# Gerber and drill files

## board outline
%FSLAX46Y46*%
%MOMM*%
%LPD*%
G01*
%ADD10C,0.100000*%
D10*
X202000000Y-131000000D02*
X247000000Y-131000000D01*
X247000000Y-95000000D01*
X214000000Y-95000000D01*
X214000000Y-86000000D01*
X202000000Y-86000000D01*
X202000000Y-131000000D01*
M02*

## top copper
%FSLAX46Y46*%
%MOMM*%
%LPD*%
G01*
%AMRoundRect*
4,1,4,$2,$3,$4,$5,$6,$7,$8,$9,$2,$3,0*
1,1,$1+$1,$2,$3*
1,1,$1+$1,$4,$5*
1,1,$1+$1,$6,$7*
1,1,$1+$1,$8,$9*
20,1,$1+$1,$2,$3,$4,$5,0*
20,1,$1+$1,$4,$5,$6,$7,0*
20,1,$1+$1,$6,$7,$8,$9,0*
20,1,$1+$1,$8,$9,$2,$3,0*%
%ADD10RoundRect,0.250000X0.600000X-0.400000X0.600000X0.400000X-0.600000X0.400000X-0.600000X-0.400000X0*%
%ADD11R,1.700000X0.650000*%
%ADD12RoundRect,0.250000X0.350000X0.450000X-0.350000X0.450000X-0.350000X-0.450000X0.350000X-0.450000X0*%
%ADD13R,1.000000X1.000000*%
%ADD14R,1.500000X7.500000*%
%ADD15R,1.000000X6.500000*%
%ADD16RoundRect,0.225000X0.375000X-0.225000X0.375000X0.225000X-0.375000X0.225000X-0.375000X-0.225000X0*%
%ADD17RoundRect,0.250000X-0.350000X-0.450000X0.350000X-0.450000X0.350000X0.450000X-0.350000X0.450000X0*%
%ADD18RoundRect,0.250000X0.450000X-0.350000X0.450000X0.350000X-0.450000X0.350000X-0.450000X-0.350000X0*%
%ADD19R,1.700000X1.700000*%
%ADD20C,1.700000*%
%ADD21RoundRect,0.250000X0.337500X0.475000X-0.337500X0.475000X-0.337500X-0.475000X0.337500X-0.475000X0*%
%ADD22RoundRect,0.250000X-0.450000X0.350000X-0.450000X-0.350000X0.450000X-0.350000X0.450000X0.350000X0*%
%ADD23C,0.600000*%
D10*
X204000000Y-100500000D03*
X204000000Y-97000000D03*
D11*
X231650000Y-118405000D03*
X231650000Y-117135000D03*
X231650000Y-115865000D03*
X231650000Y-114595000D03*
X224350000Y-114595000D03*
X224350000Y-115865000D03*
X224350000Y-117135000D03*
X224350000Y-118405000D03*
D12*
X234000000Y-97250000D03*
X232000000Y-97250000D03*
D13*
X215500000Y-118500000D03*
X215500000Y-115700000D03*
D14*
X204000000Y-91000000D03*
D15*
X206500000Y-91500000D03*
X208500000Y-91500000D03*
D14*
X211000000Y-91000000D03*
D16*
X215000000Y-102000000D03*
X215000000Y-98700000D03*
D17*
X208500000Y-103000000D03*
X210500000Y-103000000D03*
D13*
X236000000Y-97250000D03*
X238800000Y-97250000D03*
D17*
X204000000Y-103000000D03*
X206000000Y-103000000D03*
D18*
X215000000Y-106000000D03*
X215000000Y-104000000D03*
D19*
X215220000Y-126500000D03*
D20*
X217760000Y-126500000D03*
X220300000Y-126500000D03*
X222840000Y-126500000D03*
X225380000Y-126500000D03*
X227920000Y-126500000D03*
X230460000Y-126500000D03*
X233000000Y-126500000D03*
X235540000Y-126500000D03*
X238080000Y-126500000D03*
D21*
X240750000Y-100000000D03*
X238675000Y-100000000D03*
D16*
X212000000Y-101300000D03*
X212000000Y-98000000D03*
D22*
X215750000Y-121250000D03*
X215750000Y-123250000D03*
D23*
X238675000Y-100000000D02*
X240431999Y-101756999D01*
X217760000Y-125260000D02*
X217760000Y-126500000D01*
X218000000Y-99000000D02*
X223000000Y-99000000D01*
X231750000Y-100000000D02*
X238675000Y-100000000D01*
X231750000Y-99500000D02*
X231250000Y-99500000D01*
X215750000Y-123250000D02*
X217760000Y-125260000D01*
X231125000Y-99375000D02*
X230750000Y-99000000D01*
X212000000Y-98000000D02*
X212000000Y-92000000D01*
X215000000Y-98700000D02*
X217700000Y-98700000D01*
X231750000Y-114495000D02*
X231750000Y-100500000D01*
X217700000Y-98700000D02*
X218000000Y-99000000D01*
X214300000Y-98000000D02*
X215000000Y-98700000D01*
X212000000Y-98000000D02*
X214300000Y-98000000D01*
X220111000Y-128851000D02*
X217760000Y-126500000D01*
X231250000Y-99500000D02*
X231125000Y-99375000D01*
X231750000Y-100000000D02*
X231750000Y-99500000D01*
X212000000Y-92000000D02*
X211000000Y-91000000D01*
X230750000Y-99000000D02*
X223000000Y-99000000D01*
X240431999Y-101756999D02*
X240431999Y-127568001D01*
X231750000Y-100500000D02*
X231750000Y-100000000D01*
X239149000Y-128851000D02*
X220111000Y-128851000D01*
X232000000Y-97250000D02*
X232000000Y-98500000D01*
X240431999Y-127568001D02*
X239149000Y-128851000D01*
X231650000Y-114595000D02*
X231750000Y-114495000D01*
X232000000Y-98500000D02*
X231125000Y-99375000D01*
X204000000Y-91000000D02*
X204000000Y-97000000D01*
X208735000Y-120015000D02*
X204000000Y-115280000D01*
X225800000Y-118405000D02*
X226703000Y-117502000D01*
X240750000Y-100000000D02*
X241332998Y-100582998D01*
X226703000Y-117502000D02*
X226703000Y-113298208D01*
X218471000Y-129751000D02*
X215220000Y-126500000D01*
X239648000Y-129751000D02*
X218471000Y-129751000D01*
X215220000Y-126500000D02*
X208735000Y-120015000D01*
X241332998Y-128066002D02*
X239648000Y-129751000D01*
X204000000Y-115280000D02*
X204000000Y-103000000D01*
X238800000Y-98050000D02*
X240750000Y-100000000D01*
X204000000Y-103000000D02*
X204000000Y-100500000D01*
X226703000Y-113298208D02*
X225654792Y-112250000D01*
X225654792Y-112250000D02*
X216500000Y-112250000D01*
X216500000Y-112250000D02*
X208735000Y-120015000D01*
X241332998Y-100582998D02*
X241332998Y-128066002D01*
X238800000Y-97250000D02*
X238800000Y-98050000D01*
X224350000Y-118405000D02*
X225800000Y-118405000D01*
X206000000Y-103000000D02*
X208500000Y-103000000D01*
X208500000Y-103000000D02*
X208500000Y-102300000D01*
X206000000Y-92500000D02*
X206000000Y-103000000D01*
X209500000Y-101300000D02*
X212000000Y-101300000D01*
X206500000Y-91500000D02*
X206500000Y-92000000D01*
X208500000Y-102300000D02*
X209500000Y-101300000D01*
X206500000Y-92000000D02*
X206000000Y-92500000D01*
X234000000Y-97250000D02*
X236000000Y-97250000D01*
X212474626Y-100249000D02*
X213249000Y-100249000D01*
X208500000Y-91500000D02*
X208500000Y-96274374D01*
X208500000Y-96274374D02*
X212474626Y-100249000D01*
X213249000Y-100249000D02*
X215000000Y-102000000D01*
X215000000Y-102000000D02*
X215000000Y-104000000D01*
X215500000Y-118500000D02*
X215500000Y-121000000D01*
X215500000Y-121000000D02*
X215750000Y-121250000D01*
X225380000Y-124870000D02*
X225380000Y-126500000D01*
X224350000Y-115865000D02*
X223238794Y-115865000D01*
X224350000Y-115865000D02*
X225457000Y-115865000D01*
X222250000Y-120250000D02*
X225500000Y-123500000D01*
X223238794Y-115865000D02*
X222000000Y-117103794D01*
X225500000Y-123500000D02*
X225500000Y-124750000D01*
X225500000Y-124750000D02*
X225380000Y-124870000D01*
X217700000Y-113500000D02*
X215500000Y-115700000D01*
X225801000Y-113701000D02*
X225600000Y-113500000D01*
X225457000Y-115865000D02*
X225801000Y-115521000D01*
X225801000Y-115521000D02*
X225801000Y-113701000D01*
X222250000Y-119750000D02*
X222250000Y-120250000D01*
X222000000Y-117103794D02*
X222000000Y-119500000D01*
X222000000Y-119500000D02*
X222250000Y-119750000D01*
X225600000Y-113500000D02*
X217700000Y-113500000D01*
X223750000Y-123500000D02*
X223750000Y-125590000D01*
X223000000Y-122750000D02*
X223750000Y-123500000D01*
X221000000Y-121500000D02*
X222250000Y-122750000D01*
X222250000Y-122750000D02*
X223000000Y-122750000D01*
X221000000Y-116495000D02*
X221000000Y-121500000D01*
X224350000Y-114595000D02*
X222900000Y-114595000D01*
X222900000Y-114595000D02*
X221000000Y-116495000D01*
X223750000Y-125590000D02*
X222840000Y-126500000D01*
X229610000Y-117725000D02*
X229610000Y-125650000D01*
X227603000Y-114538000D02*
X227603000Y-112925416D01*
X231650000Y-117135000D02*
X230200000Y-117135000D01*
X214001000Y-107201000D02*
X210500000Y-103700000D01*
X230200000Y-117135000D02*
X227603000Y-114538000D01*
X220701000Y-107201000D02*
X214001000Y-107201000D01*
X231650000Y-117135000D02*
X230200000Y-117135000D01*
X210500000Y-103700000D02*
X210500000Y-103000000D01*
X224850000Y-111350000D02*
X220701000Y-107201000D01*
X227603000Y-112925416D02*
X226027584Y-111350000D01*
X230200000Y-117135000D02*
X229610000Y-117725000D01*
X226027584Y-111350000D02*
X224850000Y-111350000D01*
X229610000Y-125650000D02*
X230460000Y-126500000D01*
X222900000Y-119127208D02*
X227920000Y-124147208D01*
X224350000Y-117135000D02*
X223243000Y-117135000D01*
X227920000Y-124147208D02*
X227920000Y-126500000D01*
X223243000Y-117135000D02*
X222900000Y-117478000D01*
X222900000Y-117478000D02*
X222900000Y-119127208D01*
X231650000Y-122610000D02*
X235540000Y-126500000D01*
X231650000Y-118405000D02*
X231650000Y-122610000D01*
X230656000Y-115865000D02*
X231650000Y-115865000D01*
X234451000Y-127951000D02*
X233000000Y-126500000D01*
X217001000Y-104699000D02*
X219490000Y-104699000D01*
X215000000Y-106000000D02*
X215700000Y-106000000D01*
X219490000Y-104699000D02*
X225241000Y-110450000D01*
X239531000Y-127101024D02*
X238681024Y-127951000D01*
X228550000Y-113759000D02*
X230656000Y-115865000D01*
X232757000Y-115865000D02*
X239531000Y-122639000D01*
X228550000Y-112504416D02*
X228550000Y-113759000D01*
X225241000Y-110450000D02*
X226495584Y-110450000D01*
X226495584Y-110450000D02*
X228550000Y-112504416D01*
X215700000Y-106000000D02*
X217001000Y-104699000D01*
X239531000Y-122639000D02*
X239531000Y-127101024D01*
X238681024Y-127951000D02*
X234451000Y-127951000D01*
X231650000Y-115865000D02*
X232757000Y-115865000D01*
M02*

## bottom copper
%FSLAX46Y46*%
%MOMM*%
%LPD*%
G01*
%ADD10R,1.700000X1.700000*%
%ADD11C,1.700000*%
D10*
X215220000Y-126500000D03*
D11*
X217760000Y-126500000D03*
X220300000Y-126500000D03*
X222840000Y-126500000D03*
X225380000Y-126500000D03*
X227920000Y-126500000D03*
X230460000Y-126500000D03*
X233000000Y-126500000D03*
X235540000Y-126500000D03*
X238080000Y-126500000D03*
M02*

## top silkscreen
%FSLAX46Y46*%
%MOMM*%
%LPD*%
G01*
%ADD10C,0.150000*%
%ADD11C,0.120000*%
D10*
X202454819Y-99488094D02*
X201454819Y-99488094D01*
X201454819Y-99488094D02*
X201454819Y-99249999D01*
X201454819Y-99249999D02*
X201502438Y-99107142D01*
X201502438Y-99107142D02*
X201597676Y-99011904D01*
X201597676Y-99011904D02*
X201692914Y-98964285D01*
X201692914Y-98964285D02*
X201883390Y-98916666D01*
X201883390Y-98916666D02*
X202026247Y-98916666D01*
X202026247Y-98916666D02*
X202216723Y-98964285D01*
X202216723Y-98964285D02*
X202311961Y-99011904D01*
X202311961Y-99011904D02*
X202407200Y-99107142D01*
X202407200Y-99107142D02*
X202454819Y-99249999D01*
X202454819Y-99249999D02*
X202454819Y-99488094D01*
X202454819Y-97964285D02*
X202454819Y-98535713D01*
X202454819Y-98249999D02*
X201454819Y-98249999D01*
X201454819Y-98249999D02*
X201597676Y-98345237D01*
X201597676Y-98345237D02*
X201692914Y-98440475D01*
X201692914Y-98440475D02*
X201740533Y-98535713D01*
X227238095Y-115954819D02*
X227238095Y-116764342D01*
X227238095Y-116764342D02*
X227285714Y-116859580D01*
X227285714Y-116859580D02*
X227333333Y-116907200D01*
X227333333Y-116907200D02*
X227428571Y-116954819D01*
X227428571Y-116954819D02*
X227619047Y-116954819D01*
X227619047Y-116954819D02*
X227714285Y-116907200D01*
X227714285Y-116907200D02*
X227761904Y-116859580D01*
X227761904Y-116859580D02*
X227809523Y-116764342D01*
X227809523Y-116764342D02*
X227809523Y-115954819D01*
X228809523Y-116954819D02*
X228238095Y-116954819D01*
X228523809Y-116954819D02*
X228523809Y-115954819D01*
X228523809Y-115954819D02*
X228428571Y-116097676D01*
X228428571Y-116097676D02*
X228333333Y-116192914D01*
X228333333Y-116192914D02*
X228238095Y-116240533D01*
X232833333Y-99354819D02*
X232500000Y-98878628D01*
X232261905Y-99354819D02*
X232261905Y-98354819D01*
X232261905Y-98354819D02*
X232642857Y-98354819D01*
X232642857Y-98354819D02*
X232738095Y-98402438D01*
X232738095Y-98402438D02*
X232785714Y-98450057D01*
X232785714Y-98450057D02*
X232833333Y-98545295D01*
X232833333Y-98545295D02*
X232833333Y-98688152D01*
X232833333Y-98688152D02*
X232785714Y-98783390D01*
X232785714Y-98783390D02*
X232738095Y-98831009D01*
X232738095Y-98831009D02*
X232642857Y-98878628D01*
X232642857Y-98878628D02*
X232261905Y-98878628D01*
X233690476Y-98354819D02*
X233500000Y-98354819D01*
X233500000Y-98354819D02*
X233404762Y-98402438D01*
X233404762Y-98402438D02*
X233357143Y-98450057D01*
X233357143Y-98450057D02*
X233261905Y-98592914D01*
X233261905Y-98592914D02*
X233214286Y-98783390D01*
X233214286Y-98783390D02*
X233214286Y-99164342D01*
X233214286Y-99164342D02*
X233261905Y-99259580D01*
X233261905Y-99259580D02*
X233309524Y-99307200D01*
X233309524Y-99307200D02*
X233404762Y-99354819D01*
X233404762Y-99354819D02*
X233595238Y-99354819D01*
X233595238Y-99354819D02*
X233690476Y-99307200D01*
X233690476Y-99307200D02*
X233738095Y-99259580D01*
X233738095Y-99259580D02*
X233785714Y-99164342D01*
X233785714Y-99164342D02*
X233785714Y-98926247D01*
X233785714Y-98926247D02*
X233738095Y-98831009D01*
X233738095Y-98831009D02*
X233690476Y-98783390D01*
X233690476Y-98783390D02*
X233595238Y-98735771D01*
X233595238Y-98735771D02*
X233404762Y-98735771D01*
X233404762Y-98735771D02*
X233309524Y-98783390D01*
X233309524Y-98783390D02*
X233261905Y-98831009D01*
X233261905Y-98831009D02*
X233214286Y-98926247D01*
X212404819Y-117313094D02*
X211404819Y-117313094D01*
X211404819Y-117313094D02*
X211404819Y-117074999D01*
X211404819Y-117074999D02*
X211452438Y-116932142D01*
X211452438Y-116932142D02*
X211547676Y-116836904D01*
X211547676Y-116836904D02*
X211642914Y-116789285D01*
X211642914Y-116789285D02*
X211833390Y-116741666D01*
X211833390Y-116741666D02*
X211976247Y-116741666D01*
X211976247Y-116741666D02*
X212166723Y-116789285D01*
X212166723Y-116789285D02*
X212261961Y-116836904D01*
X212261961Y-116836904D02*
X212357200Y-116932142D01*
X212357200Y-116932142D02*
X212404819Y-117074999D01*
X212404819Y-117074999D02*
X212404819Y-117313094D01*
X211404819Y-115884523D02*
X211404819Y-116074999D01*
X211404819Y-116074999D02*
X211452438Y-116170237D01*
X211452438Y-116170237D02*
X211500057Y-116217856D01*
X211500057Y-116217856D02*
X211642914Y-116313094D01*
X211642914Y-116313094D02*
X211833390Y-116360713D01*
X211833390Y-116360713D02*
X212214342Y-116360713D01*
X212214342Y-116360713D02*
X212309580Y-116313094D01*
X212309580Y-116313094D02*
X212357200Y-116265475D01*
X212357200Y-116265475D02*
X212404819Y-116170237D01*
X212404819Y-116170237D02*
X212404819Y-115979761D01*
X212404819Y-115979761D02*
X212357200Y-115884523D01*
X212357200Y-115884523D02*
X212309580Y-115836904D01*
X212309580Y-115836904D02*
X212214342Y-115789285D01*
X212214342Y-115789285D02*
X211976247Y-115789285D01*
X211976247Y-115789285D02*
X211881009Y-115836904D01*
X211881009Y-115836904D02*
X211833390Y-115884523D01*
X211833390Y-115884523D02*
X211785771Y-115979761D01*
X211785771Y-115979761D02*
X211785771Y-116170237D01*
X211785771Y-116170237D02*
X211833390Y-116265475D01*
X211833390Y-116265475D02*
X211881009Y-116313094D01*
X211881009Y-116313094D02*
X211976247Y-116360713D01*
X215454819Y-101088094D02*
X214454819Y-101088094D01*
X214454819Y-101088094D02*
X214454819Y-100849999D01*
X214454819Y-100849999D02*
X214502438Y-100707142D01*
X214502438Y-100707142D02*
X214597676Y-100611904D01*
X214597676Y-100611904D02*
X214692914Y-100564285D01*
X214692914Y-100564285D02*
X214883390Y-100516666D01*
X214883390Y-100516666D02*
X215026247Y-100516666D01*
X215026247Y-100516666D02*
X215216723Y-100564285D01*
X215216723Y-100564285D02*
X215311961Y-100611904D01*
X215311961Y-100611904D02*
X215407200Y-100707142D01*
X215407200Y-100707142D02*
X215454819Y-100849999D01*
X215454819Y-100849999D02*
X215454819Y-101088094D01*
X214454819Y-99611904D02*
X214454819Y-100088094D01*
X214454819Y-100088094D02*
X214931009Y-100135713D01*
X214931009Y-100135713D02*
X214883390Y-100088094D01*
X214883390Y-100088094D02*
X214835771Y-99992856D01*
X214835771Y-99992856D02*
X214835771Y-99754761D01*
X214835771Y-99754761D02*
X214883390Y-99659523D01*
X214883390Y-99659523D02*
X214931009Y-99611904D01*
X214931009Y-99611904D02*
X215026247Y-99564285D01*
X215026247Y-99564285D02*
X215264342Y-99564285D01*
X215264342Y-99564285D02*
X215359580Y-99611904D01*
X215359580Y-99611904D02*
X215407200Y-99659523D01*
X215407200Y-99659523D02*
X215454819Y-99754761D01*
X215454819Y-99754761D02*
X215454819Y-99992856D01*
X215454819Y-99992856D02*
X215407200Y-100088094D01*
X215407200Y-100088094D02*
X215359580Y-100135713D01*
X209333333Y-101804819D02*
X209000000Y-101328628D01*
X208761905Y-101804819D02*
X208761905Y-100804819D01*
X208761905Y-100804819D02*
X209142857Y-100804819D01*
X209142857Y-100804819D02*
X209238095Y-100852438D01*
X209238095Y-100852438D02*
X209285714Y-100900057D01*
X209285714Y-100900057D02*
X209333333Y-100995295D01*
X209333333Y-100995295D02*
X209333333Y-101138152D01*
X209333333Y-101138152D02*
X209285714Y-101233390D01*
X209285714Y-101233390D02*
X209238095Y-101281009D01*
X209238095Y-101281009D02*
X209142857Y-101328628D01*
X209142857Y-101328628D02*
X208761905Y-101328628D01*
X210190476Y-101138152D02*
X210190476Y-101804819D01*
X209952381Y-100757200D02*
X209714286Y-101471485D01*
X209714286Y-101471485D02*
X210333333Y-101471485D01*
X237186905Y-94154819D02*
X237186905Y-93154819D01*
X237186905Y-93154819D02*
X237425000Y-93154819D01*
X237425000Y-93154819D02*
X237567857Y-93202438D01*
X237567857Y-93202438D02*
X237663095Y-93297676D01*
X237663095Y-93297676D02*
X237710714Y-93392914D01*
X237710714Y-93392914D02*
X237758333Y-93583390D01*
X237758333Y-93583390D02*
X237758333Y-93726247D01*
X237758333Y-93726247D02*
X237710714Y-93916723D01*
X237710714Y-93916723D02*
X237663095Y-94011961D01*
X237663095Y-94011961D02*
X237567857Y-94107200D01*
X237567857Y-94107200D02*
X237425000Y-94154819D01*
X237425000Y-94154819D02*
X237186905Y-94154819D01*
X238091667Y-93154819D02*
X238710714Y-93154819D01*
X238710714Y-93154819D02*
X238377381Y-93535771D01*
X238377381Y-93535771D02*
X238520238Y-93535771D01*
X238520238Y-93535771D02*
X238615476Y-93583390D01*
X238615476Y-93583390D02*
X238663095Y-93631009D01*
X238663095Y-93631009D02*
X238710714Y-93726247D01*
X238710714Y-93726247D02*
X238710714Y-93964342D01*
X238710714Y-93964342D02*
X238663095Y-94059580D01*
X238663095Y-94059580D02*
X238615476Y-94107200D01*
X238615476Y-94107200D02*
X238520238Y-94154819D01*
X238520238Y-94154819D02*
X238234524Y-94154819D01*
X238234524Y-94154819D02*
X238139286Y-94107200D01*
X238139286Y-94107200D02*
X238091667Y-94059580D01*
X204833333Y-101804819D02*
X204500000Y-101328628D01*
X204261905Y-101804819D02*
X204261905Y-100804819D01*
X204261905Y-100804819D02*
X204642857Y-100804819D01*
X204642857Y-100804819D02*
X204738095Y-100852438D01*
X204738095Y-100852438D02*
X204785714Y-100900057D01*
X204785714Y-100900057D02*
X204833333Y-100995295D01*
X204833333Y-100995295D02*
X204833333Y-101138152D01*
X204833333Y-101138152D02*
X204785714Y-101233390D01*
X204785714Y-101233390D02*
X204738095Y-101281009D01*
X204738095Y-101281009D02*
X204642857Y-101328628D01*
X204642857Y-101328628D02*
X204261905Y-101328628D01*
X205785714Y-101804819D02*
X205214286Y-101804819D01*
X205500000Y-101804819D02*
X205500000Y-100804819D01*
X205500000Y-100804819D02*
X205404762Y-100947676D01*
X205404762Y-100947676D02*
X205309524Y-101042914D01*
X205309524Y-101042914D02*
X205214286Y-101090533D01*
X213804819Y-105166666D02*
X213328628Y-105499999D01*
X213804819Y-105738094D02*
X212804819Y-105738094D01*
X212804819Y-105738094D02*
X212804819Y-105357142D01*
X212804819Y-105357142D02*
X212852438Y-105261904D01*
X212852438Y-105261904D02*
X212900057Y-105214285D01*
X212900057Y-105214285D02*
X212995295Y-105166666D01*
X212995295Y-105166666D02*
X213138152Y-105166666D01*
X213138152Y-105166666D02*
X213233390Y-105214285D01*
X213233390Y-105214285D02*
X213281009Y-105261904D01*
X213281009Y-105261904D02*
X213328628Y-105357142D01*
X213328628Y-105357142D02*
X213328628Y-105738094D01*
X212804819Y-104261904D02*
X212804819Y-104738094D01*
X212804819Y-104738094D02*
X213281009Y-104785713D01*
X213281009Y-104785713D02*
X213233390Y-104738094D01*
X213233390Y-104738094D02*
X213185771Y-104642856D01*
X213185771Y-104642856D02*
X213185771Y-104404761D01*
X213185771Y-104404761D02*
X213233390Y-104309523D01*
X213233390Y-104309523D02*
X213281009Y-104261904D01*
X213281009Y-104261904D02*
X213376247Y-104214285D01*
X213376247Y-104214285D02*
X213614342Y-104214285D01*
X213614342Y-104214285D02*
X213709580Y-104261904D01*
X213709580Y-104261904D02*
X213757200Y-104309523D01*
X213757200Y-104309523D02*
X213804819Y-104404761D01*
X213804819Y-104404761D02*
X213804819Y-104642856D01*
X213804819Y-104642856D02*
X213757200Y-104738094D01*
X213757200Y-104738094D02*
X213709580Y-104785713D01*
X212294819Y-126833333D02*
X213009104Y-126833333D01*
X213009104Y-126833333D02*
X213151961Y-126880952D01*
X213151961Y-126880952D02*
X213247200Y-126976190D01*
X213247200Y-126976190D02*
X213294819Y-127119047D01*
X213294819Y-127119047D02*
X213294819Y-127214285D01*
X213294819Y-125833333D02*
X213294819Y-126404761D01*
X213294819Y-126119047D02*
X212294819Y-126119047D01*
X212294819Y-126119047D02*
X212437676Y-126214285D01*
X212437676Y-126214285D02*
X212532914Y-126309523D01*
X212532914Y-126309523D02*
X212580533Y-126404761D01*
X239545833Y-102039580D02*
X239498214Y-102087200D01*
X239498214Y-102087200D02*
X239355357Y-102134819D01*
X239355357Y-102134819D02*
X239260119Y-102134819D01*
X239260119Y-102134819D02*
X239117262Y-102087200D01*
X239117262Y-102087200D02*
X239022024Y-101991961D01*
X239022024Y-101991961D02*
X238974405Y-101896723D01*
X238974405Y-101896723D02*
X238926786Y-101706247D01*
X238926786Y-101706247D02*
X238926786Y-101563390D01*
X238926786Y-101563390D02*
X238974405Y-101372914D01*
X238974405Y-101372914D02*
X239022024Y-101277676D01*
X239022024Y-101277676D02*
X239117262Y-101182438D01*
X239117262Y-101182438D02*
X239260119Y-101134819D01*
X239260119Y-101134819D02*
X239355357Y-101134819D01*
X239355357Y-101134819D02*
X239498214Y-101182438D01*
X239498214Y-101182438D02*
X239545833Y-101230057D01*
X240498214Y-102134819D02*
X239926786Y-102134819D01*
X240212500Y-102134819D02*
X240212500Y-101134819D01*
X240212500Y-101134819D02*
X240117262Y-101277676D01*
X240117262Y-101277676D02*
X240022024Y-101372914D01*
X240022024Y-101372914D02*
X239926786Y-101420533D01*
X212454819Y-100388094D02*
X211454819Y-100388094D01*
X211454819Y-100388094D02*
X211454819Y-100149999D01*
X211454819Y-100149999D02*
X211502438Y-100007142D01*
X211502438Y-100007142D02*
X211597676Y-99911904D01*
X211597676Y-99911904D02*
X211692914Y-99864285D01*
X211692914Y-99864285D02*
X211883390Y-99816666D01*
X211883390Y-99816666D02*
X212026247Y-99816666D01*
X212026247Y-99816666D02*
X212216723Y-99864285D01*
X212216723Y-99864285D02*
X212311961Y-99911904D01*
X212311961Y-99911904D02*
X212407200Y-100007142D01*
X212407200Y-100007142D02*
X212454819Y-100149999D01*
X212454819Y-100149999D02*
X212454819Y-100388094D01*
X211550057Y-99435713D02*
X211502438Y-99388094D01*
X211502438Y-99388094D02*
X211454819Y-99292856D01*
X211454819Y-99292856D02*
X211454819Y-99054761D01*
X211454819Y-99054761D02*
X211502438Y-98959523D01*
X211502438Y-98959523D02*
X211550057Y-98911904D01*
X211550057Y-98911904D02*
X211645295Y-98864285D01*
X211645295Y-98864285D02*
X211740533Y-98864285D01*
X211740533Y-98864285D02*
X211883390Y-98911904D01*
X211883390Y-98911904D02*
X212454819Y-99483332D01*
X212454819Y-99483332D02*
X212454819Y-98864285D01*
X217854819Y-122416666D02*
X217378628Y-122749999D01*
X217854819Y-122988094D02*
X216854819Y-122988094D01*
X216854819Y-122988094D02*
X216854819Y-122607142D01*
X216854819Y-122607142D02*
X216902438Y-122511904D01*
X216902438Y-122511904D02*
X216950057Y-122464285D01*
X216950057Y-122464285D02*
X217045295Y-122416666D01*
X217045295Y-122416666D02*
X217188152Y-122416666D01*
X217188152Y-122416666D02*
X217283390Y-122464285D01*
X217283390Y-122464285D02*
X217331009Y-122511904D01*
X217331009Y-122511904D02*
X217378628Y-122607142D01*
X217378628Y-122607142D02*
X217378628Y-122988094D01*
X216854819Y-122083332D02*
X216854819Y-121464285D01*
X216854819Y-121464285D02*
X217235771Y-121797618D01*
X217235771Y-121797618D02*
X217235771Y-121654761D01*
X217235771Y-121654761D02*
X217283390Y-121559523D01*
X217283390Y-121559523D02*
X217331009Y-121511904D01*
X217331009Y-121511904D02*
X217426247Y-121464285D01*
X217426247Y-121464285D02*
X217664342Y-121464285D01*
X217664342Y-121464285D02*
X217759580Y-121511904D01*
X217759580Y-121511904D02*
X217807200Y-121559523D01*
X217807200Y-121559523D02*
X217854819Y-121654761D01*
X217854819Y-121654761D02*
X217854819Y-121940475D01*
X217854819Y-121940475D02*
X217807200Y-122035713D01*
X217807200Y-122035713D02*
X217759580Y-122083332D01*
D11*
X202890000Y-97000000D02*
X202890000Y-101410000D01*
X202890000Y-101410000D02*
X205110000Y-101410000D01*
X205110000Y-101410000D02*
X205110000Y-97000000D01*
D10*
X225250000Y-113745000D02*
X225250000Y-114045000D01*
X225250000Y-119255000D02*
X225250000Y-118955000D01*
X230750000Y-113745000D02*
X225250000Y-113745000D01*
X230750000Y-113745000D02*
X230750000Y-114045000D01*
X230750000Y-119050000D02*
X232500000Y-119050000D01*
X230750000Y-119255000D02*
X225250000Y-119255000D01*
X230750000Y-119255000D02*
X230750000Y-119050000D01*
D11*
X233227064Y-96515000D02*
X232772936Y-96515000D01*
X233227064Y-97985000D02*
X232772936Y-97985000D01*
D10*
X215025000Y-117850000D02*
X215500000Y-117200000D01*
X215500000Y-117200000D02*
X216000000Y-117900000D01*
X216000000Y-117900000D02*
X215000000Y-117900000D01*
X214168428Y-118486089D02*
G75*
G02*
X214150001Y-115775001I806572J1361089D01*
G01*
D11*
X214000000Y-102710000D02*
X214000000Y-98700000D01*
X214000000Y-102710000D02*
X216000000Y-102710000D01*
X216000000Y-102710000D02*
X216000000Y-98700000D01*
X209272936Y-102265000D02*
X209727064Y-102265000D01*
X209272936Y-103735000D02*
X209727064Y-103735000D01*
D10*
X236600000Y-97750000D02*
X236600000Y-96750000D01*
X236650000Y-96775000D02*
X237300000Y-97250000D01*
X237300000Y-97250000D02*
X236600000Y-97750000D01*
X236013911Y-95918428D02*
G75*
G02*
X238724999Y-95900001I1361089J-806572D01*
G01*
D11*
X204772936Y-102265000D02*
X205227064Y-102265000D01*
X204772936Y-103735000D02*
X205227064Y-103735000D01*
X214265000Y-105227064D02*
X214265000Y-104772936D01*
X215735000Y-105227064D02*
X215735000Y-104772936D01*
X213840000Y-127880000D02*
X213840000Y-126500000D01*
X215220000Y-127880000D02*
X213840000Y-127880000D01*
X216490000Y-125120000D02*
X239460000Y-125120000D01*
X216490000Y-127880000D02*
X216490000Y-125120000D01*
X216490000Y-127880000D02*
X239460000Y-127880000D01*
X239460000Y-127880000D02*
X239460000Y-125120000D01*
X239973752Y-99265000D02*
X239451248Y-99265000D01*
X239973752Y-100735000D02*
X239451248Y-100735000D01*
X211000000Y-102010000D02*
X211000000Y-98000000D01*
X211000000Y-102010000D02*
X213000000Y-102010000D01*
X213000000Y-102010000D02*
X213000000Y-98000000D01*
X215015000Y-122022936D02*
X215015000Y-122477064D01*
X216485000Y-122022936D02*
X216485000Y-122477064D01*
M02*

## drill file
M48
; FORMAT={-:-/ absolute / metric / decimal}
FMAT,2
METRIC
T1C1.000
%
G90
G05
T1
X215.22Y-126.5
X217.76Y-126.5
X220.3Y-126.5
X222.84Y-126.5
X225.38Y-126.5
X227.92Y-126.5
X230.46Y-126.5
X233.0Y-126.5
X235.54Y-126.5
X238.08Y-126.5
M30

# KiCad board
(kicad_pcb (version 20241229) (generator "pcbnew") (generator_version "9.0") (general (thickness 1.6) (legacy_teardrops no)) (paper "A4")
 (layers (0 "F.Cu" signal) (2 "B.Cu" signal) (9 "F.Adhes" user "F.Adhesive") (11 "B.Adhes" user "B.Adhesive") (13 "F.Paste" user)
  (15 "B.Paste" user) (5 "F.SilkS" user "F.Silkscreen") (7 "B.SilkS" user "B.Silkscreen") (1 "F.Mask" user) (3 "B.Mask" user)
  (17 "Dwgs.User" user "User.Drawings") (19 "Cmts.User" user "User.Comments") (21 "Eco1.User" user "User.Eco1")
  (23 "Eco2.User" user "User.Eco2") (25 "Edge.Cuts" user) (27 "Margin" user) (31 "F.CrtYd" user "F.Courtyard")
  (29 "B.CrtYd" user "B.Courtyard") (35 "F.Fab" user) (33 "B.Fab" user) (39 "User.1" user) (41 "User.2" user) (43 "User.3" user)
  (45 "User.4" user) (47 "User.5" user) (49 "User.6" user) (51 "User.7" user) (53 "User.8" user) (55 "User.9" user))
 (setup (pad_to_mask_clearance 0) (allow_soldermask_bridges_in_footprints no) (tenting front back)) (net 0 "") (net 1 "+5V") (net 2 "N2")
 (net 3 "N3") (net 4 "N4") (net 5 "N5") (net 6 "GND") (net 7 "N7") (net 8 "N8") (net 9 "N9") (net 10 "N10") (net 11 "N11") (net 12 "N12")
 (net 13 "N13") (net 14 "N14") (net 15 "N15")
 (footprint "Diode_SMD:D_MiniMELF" (layer "F.Cu") (at 204 98.75 90)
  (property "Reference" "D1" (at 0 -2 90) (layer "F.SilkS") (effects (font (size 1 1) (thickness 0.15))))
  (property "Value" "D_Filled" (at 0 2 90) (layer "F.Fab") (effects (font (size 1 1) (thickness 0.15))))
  (fp_line (start 1.75 -1.11) (end -2.66 -1.11) (stroke (width 0.12) (type solid)) (layer "F.SilkS"))
  (fp_line (start -2.66 -1.11) (end -2.66 1.11) (stroke (width 0.12) (type solid)) (layer "F.SilkS"))
  (fp_line (start -2.66 1.11) (end 1.75 1.11) (stroke (width 0.12) (type solid)) (layer "F.SilkS"))
  (pad "1" smd roundrect (at -1.75 0 90) (size 1.3 1.7) (layers "F.Cu" "F.Mask" "F.Paste") (roundrect_rratio 0.1923076923) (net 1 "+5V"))
  (pad "2" smd roundrect (at 1.75 0 90) (size 1.3 1.7) (layers "F.Cu" "F.Mask" "F.Paste") (roundrect_rratio 0.1923076923) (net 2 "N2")))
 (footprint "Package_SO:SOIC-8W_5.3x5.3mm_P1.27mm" (layer "F.Cu") (at 228 116.5 180)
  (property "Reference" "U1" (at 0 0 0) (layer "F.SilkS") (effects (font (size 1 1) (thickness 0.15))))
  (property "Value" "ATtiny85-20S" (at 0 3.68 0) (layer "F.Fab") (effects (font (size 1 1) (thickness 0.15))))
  (fp_line (start 2.75 2.755) (end 2.75 2.455) (stroke (width 0.15) (type solid)) (layer "F.SilkS"))
  (fp_line (start 2.75 -2.755) (end 2.75 -2.455) (stroke (width 0.15) (type solid)) (layer "F.SilkS"))
  (fp_line (start -2.75 2.755) (end 2.75 2.755) (stroke (width 0.15) (type solid)) (layer "F.SilkS"))
  (fp_line (start -2.75 2.755) (end -2.75 2.455) (stroke (width 0.15) (type solid)) (layer "F.SilkS"))
  (fp_line (start -2.75 -2.55) (end -4.5 -2.55) (stroke (width 0.15) (type solid)) (layer "F.SilkS"))
  (fp_line (start -2.75 -2.755) (end 2.75 -2.755) (stroke (width 0.15) (type solid)) (layer "F.SilkS"))
  (fp_line (start -2.75 -2.755) (end -2.75 -2.55) (stroke (width 0.15) (type solid)) (layer "F.SilkS"))
  (pad "1" smd rect (at -3.65 -1.905 180) (size 1.7 0.65) (layers "F.Cu" "F.Mask" "F.Paste") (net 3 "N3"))
  (pad "2" smd rect (at -3.65 -0.635 180) (size 1.7 0.65) (layers "F.Cu" "F.Mask" "F.Paste") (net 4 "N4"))
  (pad "3" smd rect (at -3.65 0.635 180) (size 1.7 0.65) (layers "F.Cu" "F.Mask" "F.Paste") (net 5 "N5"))
  (pad "4" smd rect (at -3.65 1.905 180) (size 1.7 0.65) (layers "F.Cu" "F.Mask" "F.Paste") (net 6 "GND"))
  (pad "5" smd rect (at 3.65 1.905 180) (size 1.7 0.65) (layers "F.Cu" "F.Mask" "F.Paste") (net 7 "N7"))
  (pad "6" smd rect (at 3.65 0.635 180) (size 1.7 0.65) (layers "F.Cu" "F.Mask" "F.Paste") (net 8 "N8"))
  (pad "7" smd rect (at 3.65 -0.635 180) (size 1.7 0.65) (layers "F.Cu" "F.Mask" "F.Paste") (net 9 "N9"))
  (pad "8" smd rect (at 3.65 -1.905 180) (size 1.7 0.65) (layers "F.Cu" "F.Mask" "F.Paste") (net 1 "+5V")))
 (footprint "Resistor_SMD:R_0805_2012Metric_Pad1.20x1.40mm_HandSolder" (layer "F.Cu") (at 233 97.25 180)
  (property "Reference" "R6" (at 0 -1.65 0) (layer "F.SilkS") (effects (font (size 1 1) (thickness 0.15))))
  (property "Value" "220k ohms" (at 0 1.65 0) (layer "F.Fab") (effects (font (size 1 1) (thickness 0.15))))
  (fp_line (start -0.227064 0.735) (end 0.227064 0.735) (stroke (width 0.12) (type solid)) (layer "F.SilkS"))
  (fp_line (start -0.227064 -0.735) (end 0.227064 -0.735) (stroke (width 0.12) (type solid)) (layer "F.SilkS"))
  (pad "1" smd roundrect (at -1 0 180) (size 1.2 1.4) (layers "F.Cu" "F.Mask" "F.Paste") (roundrect_rratio 0.208333) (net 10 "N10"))
  (pad "2" smd roundrect (at 1 0 180) (size 1.2 1.4) (layers "F.Cu" "F.Mask" "F.Paste") (roundrect_rratio 0.208333) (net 6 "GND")))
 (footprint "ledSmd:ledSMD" (layer "F.Cu") (at 215.5 116.7 90)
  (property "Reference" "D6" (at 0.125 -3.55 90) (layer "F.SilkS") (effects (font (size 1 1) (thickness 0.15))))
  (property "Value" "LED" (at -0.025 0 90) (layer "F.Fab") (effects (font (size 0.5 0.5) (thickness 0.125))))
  (fp_line (start -1.15 -0.475) (end -0.5 0) (stroke (width 0.15) (type solid)) (layer "F.SilkS"))
  (fp_line (start -0.5 0) (end -1.2 0.5) (stroke (width 0.15) (type solid)) (layer "F.SilkS"))
  (fp_line (start -1.2 0.5) (end -1.2 -0.5) (stroke (width 0.15) (type solid)) (layer "F.SilkS"))
  (fp_arc (start -1.786089 -1.331572) (mid -0.435753 -2.107089) (end 0.924999 -1.349999) (stroke (width 0.15) (type solid))
   (layer "F.SilkS"))
  (pad "1" smd rect (at -1.8 0 90) (size 1 1) (layers "F.Cu" "F.Mask" "F.Paste") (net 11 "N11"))
  (pad "2" smd rect (at 1 0 90) (size 1 1) (layers "F.Cu" "F.Mask" "F.Paste") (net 8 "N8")))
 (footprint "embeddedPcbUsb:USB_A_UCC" (layer "F.Cu") (at 207.5 91.2 -90)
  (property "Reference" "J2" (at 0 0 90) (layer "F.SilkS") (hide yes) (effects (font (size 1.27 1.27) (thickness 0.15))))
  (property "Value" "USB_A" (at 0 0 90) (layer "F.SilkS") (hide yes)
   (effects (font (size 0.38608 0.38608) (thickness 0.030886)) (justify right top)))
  (pad "1" smd rect (at -0.2 3.5 270) (size 7.5 1.5) (layers "F.Cu" "F.Mask" "F.Paste") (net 2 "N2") (solder_mask_margin 0.1016))
  (pad "2" smd rect (at 0.3 1 270) (size 6.5 1) (layers "F.Cu" "F.Mask" "F.Paste") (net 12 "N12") (solder_mask_margin 0.1016))
  (pad "3" smd rect (at 0.3 -1 270) (size 6.5 1) (layers "F.Cu" "F.Mask" "F.Paste") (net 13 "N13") (solder_mask_margin 0.1016))
  (pad "4" smd rect (at -0.2 -3.5 270) (size 7.5 1.5) (layers "F.Cu" "F.Mask" "F.Paste") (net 6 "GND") (solder_mask_margin 0.1016)))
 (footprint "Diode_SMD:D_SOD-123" (layer "F.Cu") (at 215 100.35 90)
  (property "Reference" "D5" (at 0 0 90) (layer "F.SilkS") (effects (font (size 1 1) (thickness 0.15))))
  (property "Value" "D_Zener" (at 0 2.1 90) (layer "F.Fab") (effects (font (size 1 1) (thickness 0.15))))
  (fp_line (start -2.36 -1) (end 1.65 -1) (stroke (width 0.12) (type solid)) (layer "F.SilkS"))
  (fp_line (start -2.36 -1) (end -2.36 1) (stroke (width 0.12) (type solid)) (layer "F.SilkS"))
  (fp_line (start -2.36 1) (end 1.65 1) (stroke (width 0.12) (type solid)) (layer "F.SilkS"))
  (pad "1" smd roundrect (at -1.65 0 90) (size 0.9 1.2) (layers "F.Cu" "F.Mask" "F.Paste") (roundrect_rratio 0.25) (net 13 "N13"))
  (pad "2" smd roundrect (at 1.65 0 90) (size 0.9 1.2) (layers "F.Cu" "F.Mask" "F.Paste") (roundrect_rratio 0.25) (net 6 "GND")))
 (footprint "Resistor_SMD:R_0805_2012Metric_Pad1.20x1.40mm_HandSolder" (layer "F.Cu") (at 209.5 103)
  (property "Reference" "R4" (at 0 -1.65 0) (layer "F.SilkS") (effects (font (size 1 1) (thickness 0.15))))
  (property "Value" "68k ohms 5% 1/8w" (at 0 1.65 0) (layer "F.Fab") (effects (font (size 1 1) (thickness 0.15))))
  (fp_line (start -0.227064 -0.735) (end 0.227064 -0.735) (stroke (width 0.12) (type solid)) (layer "F.SilkS"))
  (fp_line (start -0.227064 0.735) (end 0.227064 0.735) (stroke (width 0.12) (type solid)) (layer "F.SilkS"))
  (pad "1" smd roundrect (at -1 0) (size 1.2 1.4) (layers "F.Cu" "F.Mask" "F.Paste") (roundrect_rratio 0.208333) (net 12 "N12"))
  (pad "2" smd roundrect (at 1 0) (size 1.2 1.4) (layers "F.Cu" "F.Mask" "F.Paste") (roundrect_rratio 0.208333) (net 4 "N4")))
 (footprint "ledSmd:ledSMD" (layer "F.Cu") (at 237.8 97.25)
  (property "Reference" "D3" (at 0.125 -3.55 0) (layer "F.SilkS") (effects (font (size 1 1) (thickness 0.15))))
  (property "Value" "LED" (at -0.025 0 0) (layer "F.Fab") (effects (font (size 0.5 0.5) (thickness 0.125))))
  (fp_line (start -1.2 0.5) (end -1.2 -0.5) (stroke (width 0.15) (type solid)) (layer "F.SilkS"))
  (fp_line (start -1.15 -0.475) (end -0.5 0) (stroke (width 0.15) (type solid)) (layer "F.SilkS"))
  (fp_line (start -0.5 0) (end -1.2 0.5) (stroke (width 0.15) (type solid)) (layer "F.SilkS"))
  (fp_arc (start -1.786089 -1.331572) (mid -0.435753 -2.107089) (end 0.924999 -1.349999) (stroke (width 0.15) (type solid))
   (layer "F.SilkS"))
  (pad "1" smd rect (at -1.8 0) (size 1 1) (layers "F.Cu" "F.Mask" "F.Paste") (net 10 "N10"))
  (pad "2" smd rect (at 1 0) (size 1 1) (layers "F.Cu" "F.Mask" "F.Paste") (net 1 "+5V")))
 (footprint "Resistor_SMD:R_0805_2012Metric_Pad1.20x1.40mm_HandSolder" (layer "F.Cu") (at 205 103)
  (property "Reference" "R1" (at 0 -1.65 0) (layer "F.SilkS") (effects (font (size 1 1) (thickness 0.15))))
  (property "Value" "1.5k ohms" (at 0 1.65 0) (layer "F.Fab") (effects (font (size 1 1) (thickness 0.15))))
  (fp_line (start -0.227064 -0.735) (end 0.227064 -0.735) (stroke (width 0.12) (type solid)) (layer "F.SilkS"))
  (fp_line (start -0.227064 0.735) (end 0.227064 0.735) (stroke (width 0.12) (type solid)) (layer "F.SilkS"))
  (pad "1" smd roundrect (at -1 0) (size 1.2 1.4) (layers "F.Cu" "F.Mask" "F.Paste") (roundrect_rratio 0.208333) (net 1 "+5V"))
  (pad "2" smd roundrect (at 1 0) (size 1.2 1.4) (layers "F.Cu" "F.Mask" "F.Paste") (roundrect_rratio 0.208333) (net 12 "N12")))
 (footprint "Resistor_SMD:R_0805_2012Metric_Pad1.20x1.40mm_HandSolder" (layer "F.Cu") (at 215 105 90)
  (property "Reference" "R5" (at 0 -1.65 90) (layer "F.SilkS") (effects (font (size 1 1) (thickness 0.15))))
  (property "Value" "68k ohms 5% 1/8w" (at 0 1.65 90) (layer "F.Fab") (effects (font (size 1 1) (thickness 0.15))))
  (fp_line (start -0.227064 -0.735) (end 0.227064 -0.735) (stroke (width 0.12) (type solid)) (layer "F.SilkS"))
  (fp_line (start -0.227064 0.735) (end 0.227064 0.735) (stroke (width 0.12) (type solid)) (layer "F.SilkS"))
  (pad "1" smd roundrect (at -1 0 90) (size 1.2 1.4) (layers "F.Cu" "F.Mask" "F.Paste") (roundrect_rratio 0.208333) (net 5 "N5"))
  (pad "2" smd roundrect (at 1 0 90) (size 1.2 1.4) (layers "F.Cu" "F.Mask" "F.Paste") (roundrect_rratio 0.208333) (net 13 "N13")))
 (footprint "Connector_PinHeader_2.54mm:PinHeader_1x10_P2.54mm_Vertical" (layer "F.Cu") (at 215.22 126.5 90)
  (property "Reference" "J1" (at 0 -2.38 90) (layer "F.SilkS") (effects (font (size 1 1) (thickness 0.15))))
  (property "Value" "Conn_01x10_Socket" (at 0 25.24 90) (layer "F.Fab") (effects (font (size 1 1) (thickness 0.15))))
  (fp_line (start -1.38 -1.38) (end 0 -1.38) (stroke (width 0.12) (type solid)) (layer "F.SilkS"))
  (fp_line (start -1.38 0) (end -1.38 -1.38) (stroke (width 0.12) (type solid)) (layer "F.SilkS"))
  (fp_line (start 1.38 1.27) (end 1.38 24.24) (stroke (width 0.12) (type solid)) (layer "F.SilkS"))
  (fp_line (start -1.38 1.27) (end 1.38 1.27) (stroke (width 0.12) (type solid)) (layer "F.SilkS"))
  (fp_line (start -1.38 1.27) (end -1.38 24.24) (stroke (width 0.12) (type solid)) (layer "F.SilkS"))
  (fp_line (start -1.38 24.24) (end 1.38 24.24) (stroke (width 0.12) (type solid)) (layer "F.SilkS"))
  (pad "1" thru_hole rect (at 0 0 90) (size 1.7 1.7) (drill 1) (layers "*.Cu" "*.Mask") (remove_unused_layers no) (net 1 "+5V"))
  (pad "2" thru_hole circle (at 0 2.54 90) (size 1.7 1.7) (drill 1) (layers "*.Cu" "*.Mask") (remove_unused_layers no) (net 6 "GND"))
  (pad "3" thru_hole circle (at 0 5.08 90) (size 1.7 1.7) (drill 1) (layers "*.Cu" "*.Mask") (remove_unused_layers no) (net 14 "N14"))
  (pad "4" thru_hole circle (at 0 7.62 90) (size 1.7 1.7) (drill 1) (layers "*.Cu" "*.Mask") (remove_unused_layers no) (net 7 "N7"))
  (pad "5" thru_hole circle (at 0 10.16 90) (size 1.7 1.7) (drill 1) (layers "*.Cu" "*.Mask") (remove_unused_layers no) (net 8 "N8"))
  (pad "6" thru_hole circle (at 0 12.7 90) (size 1.7 1.7) (drill 1) (layers "*.Cu" "*.Mask") (remove_unused_layers no) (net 9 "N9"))
  (pad "7" thru_hole circle (at 0 15.24 90) (size 1.7 1.7) (drill 1) (layers "*.Cu" "*.Mask") (remove_unused_layers no) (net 4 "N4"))
  (pad "8" thru_hole circle (at 0 17.78 90) (size 1.7 1.7) (drill 1) (layers "*.Cu" "*.Mask") (remove_unused_layers no) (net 5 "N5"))
  (pad "9" thru_hole circle (at 0 20.32 90) (size 1.7 1.7) (drill 1) (layers "*.Cu" "*.Mask") (remove_unused_layers no) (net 3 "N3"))
  (pad "10" thru_hole circle (at 0 22.86 90) (size 1.7 1.7) (drill 1) (layers "*.Cu" "*.Mask") (remove_unused_layers no) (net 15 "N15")))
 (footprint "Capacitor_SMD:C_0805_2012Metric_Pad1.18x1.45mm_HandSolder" (layer "F.Cu") (at 239.7125 100 180)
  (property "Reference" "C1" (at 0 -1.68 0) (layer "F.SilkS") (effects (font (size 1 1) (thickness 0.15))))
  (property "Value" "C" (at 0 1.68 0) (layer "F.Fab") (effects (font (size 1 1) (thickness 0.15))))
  (fp_line (start -0.261252 0.735) (end 0.261252 0.735) (stroke (width 0.12) (type solid)) (layer "F.SilkS"))
  (fp_line (start -0.261252 -0.735) (end 0.261252 -0.735) (stroke (width 0.12) (type solid)) (layer "F.SilkS"))
  (pad "1" smd roundrect (at -1.0375 0 180) (size 1.175 1.45) (layers "F.Cu" "F.Mask" "F.Paste") (roundrect_rratio 0.212766) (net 1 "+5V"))
  (pad "2" smd roundrect (at 1.0375 0 180) (size 1.175 1.45) (layers "F.Cu" "F.Mask" "F.Paste") (roundrect_rratio 0.212766) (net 6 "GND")))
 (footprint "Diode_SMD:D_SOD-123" (layer "F.Cu") (at 212 99.65 90)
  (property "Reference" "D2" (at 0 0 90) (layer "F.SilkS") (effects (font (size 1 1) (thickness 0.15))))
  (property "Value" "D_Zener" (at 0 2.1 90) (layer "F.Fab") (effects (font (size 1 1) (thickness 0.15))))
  (fp_line (start -2.36 -1) (end 1.65 -1) (stroke (width 0.12) (type solid)) (layer "F.SilkS"))
  (fp_line (start -2.36 -1) (end -2.36 1) (stroke (width 0.12) (type solid)) (layer "F.SilkS"))
  (fp_line (start -2.36 1) (end 1.65 1) (stroke (width 0.12) (type solid)) (layer "F.SilkS"))
  (pad "1" smd roundrect (at -1.65 0 90) (size 0.9 1.2) (layers "F.Cu" "F.Mask" "F.Paste") (roundrect_rratio 0.25) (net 12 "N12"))
  (pad "2" smd roundrect (at 1.65 0 90) (size 0.9 1.2) (layers "F.Cu" "F.Mask" "F.Paste") (roundrect_rratio 0.25) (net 6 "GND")))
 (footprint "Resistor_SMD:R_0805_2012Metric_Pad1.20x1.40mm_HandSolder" (layer "F.Cu") (at 215.75 122.25 -90)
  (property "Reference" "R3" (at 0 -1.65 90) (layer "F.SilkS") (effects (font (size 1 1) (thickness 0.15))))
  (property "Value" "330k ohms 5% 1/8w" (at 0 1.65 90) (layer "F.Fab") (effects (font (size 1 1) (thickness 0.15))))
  (fp_line (start -0.227064 0.735) (end 0.227064 0.735) (stroke (width 0.12) (type solid)) (layer "F.SilkS"))
  (fp_line (start -0.227064 -0.735) (end 0.227064 -0.735) (stroke (width 0.12) (type solid)) (layer "F.SilkS"))
  (pad "1" smd roundrect (at -1 0 270) (size 1.2 1.4) (layers "F.Cu" "F.Mask" "F.Paste") (roundrect_rratio 0.208333) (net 11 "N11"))
  (pad "2" smd roundrect (at 1 0 270) (size 1.2 1.4) (layers "F.Cu" "F.Mask" "F.Paste") (roundrect_rratio 0.208333) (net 6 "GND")))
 (gr_poly
  (pts (xy 202 131) (xy 247 131) (xy 247 95) (xy 214 95) (xy 214 86) (xy 202 86)) (stroke (width 0.1) (type solid)) (fill no)
  (layer "Edge.Cuts"))
 (segment (start 238.675 100) (end 240.431999 101.756999) (width 0.6) (layer "F.Cu") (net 6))
 (segment (start 217.76 125.26) (end 217.76 126.5) (width 0.6) (layer "F.Cu") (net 6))
 (segment (start 218 99) (end 223 99) (width 0.6) (layer "F.Cu") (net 6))
 (segment (start 231.75 100) (end 238.675 100) (width 0.6) (layer "F.Cu") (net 6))
 (segment (start 231.75 99.5) (end 231.25 99.5) (width 0.6) (layer "F.Cu") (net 6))
 (segment (start 215.75 123.25) (end 217.76 125.26) (width 0.6) (layer "F.Cu") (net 6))
 (segment (start 231.125 99.375) (end 230.75 99) (width 0.6) (layer "F.Cu") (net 6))
 (segment (start 212 98) (end 212 92) (width 0.6) (layer "F.Cu") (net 6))
 (segment (start 215 98.7) (end 217.7 98.7) (width 0.6) (layer "F.Cu") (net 6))
 (segment (start 231.75 114.495) (end 231.75 100.5) (width 0.6) (layer "F.Cu") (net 6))
 (segment (start 217.7 98.7) (end 218 99) (width 0.6) (layer "F.Cu") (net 6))
 (segment (start 214.3 98) (end 215 98.7) (width 0.6) (layer "F.Cu") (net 6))
 (segment (start 212 98) (end 214.3 98) (width 0.6) (layer "F.Cu") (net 6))
 (segment (start 220.111 128.851) (end 217.76 126.5) (width 0.6) (layer "F.Cu") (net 6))
 (segment (start 231.25 99.5) (end 231.125 99.375) (width 0.6) (layer "F.Cu") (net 6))
 (segment (start 231.75 100) (end 231.75 99.5) (width 0.6) (layer "F.Cu") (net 6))
 (segment (start 212 92) (end 211 91) (width 0.6) (layer "F.Cu") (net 6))
 (segment (start 230.75 99) (end 223 99) (width 0.6) (layer "F.Cu") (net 6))
 (segment (start 240.431999 101.756999) (end 240.431999 127.568001) (width 0.6) (layer "F.Cu") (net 6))
 (segment (start 231.75 100.5) (end 231.75 100) (width 0.6) (layer "F.Cu") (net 6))
 (segment (start 239.149 128.851) (end 220.111 128.851) (width 0.6) (layer "F.Cu") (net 6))
 (segment (start 232 97.25) (end 232 98.5) (width 0.6) (layer "F.Cu") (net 6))
 (segment (start 240.431999 127.568001) (end 239.149 128.851) (width 0.6) (layer "F.Cu") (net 6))
 (segment (start 231.65 114.595) (end 231.75 114.495) (width 0.6) (layer "F.Cu") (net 6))
 (segment (start 232 98.5) (end 231.125 99.375) (width 0.6) (layer "F.Cu") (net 6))
 (segment (start 204 91) (end 204 97) (width 0.6) (layer "F.Cu") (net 2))
 (segment (start 208.735 120.015) (end 204 115.28) (width 0.6) (layer "F.Cu") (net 1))
 (segment (start 225.8 118.405) (end 226.703 117.502) (width 0.6) (layer "F.Cu") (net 1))
 (segment (start 240.75 100) (end 241.332998 100.582998) (width 0.6) (layer "F.Cu") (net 1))
 (segment (start 226.703 117.502) (end 226.703 113.298208) (width 0.6) (layer "F.Cu") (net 1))
 (segment (start 218.471 129.751) (end 215.22 126.5) (width 0.6) (layer "F.Cu") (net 1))
 (segment (start 239.648 129.751) (end 218.471 129.751) (width 0.6) (layer "F.Cu") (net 1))
 (segment (start 215.22 126.5) (end 208.735 120.015) (width 0.6) (layer "F.Cu") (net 1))
 (segment (start 241.332998 128.066002) (end 239.648 129.751) (width 0.6) (layer "F.Cu") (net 1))
 (segment (start 204 115.28) (end 204 103) (width 0.6) (layer "F.Cu") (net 1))
 (segment (start 238.8 98.05) (end 240.75 100) (width 0.6) (layer "F.Cu") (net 1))
 (segment (start 204 103) (end 204 100.5) (width 0.6) (layer "F.Cu") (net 1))
 (segment (start 226.703 113.298208) (end 225.654792 112.25) (width 0.6) (layer "F.Cu") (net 1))
 (segment (start 225.654792 112.25) (end 216.5 112.25) (width 0.6) (layer "F.Cu") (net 1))
 (segment (start 216.5 112.25) (end 208.735 120.015) (width 0.6) (layer "F.Cu") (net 1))
 (segment (start 241.332998 100.582998) (end 241.332998 128.066002) (width 0.6) (layer "F.Cu") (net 1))
 (segment (start 238.8 97.25) (end 238.8 98.05) (width 0.6) (layer "F.Cu") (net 1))
 (segment (start 224.35 118.405) (end 225.8 118.405) (width 0.6) (layer "F.Cu") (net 1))
 (segment (start 206 103) (end 208.5 103) (width 0.6) (layer "F.Cu") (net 12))
 (segment (start 208.5 103) (end 208.5 102.3) (width 0.6) (layer "F.Cu") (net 12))
 (segment (start 206 92.5) (end 206 103) (width 0.6) (layer "F.Cu") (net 12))
 (segment (start 209.5 101.3) (end 212 101.3) (width 0.6) (layer "F.Cu") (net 12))
 (segment (start 206.5 91.5) (end 206.5 92) (width 0.6) (layer "F.Cu") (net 12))
 (segment (start 208.5 102.3) (end 209.5 101.3) (width 0.6) (layer "F.Cu") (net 12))
 (segment (start 206.5 92) (end 206 92.5) (width 0.6) (layer "F.Cu") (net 12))
 (segment (start 234 97.25) (end 236 97.25) (width 0.6) (layer "F.Cu") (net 10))
 (segment (start 212.474626 100.249) (end 213.249 100.249) (width 0.6) (layer "F.Cu") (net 13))
 (segment (start 208.5 91.5) (end 208.5 96.274374) (width 0.6) (layer "F.Cu") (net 13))
 (segment (start 208.5 96.274374) (end 212.474626 100.249) (width 0.6) (layer "F.Cu") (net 13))
 (segment (start 213.249 100.249) (end 215 102) (width 0.6) (layer "F.Cu") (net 13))
 (segment (start 215 102) (end 215 104) (width 0.6) (layer "F.Cu") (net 13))
 (segment (start 215.5 118.5) (end 215.5 121) (width 0.6) (layer "F.Cu") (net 11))
 (segment (start 215.5 121) (end 215.75 121.25) (width 0.6) (layer "F.Cu") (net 11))
 (segment (start 225.38 124.87) (end 225.38 126.5) (width 0.6) (layer "F.Cu") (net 8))
 (segment (start 224.35 115.865) (end 223.238794 115.865) (width 0.6) (layer "F.Cu") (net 8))
 (segment (start 224.35 115.865) (end 225.457 115.865) (width 0.6) (layer "F.Cu") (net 8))
 (segment (start 222.25 120.25) (end 225.5 123.5) (width 0.6) (layer "F.Cu") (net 8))
 (segment (start 223.238794 115.865) (end 222 117.103794) (width 0.6) (layer "F.Cu") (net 8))
 (segment (start 225.5 123.5) (end 225.5 124.75) (width 0.6) (layer "F.Cu") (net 8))
 (segment (start 225.5 124.75) (end 225.38 124.87) (width 0.6) (layer "F.Cu") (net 8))
 (segment (start 217.7 113.5) (end 215.5 115.7) (width 0.6) (layer "F.Cu") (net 8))
 (segment (start 225.801 113.701) (end 225.6 113.5) (width 0.6) (layer "F.Cu") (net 8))
 (segment (start 225.457 115.865) (end 225.801 115.521) (width 0.6) (layer "F.Cu") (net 8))
 (segment (start 225.801 115.521) (end 225.801 113.701) (width 0.6) (layer "F.Cu") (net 8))
 (segment (start 222.25 119.75) (end 222.25 120.25) (width 0.6) (layer "F.Cu") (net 8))
 (segment (start 222 117.103794) (end 222 119.5) (width 0.6) (layer "F.Cu") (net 8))
 (segment (start 222 119.5) (end 222.25 119.75) (width 0.6) (layer "F.Cu") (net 8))
 (segment (start 225.6 113.5) (end 217.7 113.5) (width 0.6) (layer "F.Cu") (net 8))
 (segment (start 223.75 123.5) (end 223.75 125.59) (width 0.6) (layer "F.Cu") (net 7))
 (segment (start 223 122.75) (end 223.75 123.5) (width 0.6) (layer "F.Cu") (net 7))
 (segment (start 221 121.5) (end 222.25 122.75) (width 0.6) (layer "F.Cu") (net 7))
 (segment (start 222.25 122.75) (end 223 122.75) (width 0.6) (layer "F.Cu") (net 7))
 (segment (start 221 116.495) (end 221 121.5) (width 0.6) (layer "F.Cu") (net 7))
 (segment (start 224.35 114.595) (end 222.9 114.595) (width 0.6) (layer "F.Cu") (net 7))
 (segment (start 222.9 114.595) (end 221 116.495) (width 0.6) (layer "F.Cu") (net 7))
 (segment (start 223.75 125.59) (end 222.84 126.5) (width 0.6) (layer "F.Cu") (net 7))
 (segment (start 229.61 117.725) (end 229.61 125.65) (width 0.6) (layer "F.Cu") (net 4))
 (segment (start 227.603 114.538) (end 227.603 112.925416) (width 0.6) (layer "F.Cu") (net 4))
 (segment (start 231.65 117.135) (end 230.2 117.135) (width 0.6) (layer "F.Cu") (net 4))
 (segment (start 214.001 107.201) (end 210.5 103.7) (width 0.6) (layer "F.Cu") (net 4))
 (segment (start 230.2 117.135) (end 227.603 114.538) (width 0.6) (layer "F.Cu") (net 4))
 (segment (start 220.701 107.201) (end 214.001 107.201) (width 0.6) (layer "F.Cu") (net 4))
 (segment (start 231.65 117.135) (end 230.2 117.135) (width 0.6) (layer "F.Cu") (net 4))
 (segment (start 210.5 103.7) (end 210.5 103) (width 0.6) (layer "F.Cu") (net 4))
 (segment (start 224.85 111.35) (end 220.701 107.201) (width 0.6) (layer "F.Cu") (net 4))
 (segment (start 227.603 112.925416) (end 226.027584 111.35) (width 0.6) (layer "F.Cu") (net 4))
 (segment (start 230.2 117.135) (end 229.61 117.725) (width 0.6) (layer "F.Cu") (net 4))
 (segment (start 226.027584 111.35) (end 224.85 111.35) (width 0.6) (layer "F.Cu") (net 4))
 (segment (start 229.61 125.65) (end 230.46 126.5) (width 0.6) (layer "F.Cu") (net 4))
 (segment (start 222.9 119.127208) (end 227.92 124.147208) (width 0.6) (layer "F.Cu") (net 9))
 (segment (start 224.35 117.135) (end 223.243 117.135) (width 0.6) (layer "F.Cu") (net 9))
 (segment (start 227.92 124.147208) (end 227.92 126.5) (width 0.6) (layer "F.Cu") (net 9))
 (segment (start 223.243 117.135) (end 222.9 117.478) (width 0.6) (layer "F.Cu") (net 9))
 (segment (start 222.9 117.478) (end 222.9 119.127208) (width 0.6) (layer "F.Cu") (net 9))
 (segment (start 231.65 122.61) (end 235.54 126.5) (width 0.6) (layer "F.Cu") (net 3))
 (segment (start 231.65 118.405) (end 231.65 122.61) (width 0.6) (layer "F.Cu") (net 3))
 (segment (start 230.656 115.865) (end 231.65 115.865) (width 0.6) (layer "F.Cu") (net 5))
 (segment (start 234.451 127.951) (end 233 126.5) (width 0.6) (layer "F.Cu") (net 5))
 (segment (start 217.001 104.699) (end 219.49 104.699) (width 0.6) (layer "F.Cu") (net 5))
 (segment (start 215 106) (end 215.7 106) (width 0.6) (layer "F.Cu") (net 5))
 (segment (start 219.49 104.699) (end 225.241 110.45) (width 0.6) (layer "F.Cu") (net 5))
 (segment (start 239.531 127.101024) (end 238.681024 127.951) (width 0.6) (layer "F.Cu") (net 5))
 (segment (start 228.55 113.759) (end 230.656 115.865) (width 0.6) (layer "F.Cu") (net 5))
 (segment (start 232.757 115.865) (end 239.531 122.639) (width 0.6) (layer "F.Cu") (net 5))
 (segment (start 228.55 112.504416) (end 228.55 113.759) (width 0.6) (layer "F.Cu") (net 5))
 (segment (start 225.241 110.45) (end 226.495584 110.45) (width 0.6) (layer "F.Cu") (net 5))
 (segment (start 226.495584 110.45) (end 228.55 112.504416) (width 0.6) (layer "F.Cu") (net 5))
 (segment (start 215.7 106) (end 217.001 104.699) (width 0.6) (layer "F.Cu") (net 5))
 (segment (start 239.531 122.639) (end 239.531 127.101024) (width 0.6) (layer "F.Cu") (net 5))
 (segment (start 238.681024 127.951) (end 234.451 127.951) (width 0.6) (layer "F.Cu") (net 5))
 (segment (start 231.65 115.865) (end 232.757 115.865) (width 0.6) (layer "F.Cu") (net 5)))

